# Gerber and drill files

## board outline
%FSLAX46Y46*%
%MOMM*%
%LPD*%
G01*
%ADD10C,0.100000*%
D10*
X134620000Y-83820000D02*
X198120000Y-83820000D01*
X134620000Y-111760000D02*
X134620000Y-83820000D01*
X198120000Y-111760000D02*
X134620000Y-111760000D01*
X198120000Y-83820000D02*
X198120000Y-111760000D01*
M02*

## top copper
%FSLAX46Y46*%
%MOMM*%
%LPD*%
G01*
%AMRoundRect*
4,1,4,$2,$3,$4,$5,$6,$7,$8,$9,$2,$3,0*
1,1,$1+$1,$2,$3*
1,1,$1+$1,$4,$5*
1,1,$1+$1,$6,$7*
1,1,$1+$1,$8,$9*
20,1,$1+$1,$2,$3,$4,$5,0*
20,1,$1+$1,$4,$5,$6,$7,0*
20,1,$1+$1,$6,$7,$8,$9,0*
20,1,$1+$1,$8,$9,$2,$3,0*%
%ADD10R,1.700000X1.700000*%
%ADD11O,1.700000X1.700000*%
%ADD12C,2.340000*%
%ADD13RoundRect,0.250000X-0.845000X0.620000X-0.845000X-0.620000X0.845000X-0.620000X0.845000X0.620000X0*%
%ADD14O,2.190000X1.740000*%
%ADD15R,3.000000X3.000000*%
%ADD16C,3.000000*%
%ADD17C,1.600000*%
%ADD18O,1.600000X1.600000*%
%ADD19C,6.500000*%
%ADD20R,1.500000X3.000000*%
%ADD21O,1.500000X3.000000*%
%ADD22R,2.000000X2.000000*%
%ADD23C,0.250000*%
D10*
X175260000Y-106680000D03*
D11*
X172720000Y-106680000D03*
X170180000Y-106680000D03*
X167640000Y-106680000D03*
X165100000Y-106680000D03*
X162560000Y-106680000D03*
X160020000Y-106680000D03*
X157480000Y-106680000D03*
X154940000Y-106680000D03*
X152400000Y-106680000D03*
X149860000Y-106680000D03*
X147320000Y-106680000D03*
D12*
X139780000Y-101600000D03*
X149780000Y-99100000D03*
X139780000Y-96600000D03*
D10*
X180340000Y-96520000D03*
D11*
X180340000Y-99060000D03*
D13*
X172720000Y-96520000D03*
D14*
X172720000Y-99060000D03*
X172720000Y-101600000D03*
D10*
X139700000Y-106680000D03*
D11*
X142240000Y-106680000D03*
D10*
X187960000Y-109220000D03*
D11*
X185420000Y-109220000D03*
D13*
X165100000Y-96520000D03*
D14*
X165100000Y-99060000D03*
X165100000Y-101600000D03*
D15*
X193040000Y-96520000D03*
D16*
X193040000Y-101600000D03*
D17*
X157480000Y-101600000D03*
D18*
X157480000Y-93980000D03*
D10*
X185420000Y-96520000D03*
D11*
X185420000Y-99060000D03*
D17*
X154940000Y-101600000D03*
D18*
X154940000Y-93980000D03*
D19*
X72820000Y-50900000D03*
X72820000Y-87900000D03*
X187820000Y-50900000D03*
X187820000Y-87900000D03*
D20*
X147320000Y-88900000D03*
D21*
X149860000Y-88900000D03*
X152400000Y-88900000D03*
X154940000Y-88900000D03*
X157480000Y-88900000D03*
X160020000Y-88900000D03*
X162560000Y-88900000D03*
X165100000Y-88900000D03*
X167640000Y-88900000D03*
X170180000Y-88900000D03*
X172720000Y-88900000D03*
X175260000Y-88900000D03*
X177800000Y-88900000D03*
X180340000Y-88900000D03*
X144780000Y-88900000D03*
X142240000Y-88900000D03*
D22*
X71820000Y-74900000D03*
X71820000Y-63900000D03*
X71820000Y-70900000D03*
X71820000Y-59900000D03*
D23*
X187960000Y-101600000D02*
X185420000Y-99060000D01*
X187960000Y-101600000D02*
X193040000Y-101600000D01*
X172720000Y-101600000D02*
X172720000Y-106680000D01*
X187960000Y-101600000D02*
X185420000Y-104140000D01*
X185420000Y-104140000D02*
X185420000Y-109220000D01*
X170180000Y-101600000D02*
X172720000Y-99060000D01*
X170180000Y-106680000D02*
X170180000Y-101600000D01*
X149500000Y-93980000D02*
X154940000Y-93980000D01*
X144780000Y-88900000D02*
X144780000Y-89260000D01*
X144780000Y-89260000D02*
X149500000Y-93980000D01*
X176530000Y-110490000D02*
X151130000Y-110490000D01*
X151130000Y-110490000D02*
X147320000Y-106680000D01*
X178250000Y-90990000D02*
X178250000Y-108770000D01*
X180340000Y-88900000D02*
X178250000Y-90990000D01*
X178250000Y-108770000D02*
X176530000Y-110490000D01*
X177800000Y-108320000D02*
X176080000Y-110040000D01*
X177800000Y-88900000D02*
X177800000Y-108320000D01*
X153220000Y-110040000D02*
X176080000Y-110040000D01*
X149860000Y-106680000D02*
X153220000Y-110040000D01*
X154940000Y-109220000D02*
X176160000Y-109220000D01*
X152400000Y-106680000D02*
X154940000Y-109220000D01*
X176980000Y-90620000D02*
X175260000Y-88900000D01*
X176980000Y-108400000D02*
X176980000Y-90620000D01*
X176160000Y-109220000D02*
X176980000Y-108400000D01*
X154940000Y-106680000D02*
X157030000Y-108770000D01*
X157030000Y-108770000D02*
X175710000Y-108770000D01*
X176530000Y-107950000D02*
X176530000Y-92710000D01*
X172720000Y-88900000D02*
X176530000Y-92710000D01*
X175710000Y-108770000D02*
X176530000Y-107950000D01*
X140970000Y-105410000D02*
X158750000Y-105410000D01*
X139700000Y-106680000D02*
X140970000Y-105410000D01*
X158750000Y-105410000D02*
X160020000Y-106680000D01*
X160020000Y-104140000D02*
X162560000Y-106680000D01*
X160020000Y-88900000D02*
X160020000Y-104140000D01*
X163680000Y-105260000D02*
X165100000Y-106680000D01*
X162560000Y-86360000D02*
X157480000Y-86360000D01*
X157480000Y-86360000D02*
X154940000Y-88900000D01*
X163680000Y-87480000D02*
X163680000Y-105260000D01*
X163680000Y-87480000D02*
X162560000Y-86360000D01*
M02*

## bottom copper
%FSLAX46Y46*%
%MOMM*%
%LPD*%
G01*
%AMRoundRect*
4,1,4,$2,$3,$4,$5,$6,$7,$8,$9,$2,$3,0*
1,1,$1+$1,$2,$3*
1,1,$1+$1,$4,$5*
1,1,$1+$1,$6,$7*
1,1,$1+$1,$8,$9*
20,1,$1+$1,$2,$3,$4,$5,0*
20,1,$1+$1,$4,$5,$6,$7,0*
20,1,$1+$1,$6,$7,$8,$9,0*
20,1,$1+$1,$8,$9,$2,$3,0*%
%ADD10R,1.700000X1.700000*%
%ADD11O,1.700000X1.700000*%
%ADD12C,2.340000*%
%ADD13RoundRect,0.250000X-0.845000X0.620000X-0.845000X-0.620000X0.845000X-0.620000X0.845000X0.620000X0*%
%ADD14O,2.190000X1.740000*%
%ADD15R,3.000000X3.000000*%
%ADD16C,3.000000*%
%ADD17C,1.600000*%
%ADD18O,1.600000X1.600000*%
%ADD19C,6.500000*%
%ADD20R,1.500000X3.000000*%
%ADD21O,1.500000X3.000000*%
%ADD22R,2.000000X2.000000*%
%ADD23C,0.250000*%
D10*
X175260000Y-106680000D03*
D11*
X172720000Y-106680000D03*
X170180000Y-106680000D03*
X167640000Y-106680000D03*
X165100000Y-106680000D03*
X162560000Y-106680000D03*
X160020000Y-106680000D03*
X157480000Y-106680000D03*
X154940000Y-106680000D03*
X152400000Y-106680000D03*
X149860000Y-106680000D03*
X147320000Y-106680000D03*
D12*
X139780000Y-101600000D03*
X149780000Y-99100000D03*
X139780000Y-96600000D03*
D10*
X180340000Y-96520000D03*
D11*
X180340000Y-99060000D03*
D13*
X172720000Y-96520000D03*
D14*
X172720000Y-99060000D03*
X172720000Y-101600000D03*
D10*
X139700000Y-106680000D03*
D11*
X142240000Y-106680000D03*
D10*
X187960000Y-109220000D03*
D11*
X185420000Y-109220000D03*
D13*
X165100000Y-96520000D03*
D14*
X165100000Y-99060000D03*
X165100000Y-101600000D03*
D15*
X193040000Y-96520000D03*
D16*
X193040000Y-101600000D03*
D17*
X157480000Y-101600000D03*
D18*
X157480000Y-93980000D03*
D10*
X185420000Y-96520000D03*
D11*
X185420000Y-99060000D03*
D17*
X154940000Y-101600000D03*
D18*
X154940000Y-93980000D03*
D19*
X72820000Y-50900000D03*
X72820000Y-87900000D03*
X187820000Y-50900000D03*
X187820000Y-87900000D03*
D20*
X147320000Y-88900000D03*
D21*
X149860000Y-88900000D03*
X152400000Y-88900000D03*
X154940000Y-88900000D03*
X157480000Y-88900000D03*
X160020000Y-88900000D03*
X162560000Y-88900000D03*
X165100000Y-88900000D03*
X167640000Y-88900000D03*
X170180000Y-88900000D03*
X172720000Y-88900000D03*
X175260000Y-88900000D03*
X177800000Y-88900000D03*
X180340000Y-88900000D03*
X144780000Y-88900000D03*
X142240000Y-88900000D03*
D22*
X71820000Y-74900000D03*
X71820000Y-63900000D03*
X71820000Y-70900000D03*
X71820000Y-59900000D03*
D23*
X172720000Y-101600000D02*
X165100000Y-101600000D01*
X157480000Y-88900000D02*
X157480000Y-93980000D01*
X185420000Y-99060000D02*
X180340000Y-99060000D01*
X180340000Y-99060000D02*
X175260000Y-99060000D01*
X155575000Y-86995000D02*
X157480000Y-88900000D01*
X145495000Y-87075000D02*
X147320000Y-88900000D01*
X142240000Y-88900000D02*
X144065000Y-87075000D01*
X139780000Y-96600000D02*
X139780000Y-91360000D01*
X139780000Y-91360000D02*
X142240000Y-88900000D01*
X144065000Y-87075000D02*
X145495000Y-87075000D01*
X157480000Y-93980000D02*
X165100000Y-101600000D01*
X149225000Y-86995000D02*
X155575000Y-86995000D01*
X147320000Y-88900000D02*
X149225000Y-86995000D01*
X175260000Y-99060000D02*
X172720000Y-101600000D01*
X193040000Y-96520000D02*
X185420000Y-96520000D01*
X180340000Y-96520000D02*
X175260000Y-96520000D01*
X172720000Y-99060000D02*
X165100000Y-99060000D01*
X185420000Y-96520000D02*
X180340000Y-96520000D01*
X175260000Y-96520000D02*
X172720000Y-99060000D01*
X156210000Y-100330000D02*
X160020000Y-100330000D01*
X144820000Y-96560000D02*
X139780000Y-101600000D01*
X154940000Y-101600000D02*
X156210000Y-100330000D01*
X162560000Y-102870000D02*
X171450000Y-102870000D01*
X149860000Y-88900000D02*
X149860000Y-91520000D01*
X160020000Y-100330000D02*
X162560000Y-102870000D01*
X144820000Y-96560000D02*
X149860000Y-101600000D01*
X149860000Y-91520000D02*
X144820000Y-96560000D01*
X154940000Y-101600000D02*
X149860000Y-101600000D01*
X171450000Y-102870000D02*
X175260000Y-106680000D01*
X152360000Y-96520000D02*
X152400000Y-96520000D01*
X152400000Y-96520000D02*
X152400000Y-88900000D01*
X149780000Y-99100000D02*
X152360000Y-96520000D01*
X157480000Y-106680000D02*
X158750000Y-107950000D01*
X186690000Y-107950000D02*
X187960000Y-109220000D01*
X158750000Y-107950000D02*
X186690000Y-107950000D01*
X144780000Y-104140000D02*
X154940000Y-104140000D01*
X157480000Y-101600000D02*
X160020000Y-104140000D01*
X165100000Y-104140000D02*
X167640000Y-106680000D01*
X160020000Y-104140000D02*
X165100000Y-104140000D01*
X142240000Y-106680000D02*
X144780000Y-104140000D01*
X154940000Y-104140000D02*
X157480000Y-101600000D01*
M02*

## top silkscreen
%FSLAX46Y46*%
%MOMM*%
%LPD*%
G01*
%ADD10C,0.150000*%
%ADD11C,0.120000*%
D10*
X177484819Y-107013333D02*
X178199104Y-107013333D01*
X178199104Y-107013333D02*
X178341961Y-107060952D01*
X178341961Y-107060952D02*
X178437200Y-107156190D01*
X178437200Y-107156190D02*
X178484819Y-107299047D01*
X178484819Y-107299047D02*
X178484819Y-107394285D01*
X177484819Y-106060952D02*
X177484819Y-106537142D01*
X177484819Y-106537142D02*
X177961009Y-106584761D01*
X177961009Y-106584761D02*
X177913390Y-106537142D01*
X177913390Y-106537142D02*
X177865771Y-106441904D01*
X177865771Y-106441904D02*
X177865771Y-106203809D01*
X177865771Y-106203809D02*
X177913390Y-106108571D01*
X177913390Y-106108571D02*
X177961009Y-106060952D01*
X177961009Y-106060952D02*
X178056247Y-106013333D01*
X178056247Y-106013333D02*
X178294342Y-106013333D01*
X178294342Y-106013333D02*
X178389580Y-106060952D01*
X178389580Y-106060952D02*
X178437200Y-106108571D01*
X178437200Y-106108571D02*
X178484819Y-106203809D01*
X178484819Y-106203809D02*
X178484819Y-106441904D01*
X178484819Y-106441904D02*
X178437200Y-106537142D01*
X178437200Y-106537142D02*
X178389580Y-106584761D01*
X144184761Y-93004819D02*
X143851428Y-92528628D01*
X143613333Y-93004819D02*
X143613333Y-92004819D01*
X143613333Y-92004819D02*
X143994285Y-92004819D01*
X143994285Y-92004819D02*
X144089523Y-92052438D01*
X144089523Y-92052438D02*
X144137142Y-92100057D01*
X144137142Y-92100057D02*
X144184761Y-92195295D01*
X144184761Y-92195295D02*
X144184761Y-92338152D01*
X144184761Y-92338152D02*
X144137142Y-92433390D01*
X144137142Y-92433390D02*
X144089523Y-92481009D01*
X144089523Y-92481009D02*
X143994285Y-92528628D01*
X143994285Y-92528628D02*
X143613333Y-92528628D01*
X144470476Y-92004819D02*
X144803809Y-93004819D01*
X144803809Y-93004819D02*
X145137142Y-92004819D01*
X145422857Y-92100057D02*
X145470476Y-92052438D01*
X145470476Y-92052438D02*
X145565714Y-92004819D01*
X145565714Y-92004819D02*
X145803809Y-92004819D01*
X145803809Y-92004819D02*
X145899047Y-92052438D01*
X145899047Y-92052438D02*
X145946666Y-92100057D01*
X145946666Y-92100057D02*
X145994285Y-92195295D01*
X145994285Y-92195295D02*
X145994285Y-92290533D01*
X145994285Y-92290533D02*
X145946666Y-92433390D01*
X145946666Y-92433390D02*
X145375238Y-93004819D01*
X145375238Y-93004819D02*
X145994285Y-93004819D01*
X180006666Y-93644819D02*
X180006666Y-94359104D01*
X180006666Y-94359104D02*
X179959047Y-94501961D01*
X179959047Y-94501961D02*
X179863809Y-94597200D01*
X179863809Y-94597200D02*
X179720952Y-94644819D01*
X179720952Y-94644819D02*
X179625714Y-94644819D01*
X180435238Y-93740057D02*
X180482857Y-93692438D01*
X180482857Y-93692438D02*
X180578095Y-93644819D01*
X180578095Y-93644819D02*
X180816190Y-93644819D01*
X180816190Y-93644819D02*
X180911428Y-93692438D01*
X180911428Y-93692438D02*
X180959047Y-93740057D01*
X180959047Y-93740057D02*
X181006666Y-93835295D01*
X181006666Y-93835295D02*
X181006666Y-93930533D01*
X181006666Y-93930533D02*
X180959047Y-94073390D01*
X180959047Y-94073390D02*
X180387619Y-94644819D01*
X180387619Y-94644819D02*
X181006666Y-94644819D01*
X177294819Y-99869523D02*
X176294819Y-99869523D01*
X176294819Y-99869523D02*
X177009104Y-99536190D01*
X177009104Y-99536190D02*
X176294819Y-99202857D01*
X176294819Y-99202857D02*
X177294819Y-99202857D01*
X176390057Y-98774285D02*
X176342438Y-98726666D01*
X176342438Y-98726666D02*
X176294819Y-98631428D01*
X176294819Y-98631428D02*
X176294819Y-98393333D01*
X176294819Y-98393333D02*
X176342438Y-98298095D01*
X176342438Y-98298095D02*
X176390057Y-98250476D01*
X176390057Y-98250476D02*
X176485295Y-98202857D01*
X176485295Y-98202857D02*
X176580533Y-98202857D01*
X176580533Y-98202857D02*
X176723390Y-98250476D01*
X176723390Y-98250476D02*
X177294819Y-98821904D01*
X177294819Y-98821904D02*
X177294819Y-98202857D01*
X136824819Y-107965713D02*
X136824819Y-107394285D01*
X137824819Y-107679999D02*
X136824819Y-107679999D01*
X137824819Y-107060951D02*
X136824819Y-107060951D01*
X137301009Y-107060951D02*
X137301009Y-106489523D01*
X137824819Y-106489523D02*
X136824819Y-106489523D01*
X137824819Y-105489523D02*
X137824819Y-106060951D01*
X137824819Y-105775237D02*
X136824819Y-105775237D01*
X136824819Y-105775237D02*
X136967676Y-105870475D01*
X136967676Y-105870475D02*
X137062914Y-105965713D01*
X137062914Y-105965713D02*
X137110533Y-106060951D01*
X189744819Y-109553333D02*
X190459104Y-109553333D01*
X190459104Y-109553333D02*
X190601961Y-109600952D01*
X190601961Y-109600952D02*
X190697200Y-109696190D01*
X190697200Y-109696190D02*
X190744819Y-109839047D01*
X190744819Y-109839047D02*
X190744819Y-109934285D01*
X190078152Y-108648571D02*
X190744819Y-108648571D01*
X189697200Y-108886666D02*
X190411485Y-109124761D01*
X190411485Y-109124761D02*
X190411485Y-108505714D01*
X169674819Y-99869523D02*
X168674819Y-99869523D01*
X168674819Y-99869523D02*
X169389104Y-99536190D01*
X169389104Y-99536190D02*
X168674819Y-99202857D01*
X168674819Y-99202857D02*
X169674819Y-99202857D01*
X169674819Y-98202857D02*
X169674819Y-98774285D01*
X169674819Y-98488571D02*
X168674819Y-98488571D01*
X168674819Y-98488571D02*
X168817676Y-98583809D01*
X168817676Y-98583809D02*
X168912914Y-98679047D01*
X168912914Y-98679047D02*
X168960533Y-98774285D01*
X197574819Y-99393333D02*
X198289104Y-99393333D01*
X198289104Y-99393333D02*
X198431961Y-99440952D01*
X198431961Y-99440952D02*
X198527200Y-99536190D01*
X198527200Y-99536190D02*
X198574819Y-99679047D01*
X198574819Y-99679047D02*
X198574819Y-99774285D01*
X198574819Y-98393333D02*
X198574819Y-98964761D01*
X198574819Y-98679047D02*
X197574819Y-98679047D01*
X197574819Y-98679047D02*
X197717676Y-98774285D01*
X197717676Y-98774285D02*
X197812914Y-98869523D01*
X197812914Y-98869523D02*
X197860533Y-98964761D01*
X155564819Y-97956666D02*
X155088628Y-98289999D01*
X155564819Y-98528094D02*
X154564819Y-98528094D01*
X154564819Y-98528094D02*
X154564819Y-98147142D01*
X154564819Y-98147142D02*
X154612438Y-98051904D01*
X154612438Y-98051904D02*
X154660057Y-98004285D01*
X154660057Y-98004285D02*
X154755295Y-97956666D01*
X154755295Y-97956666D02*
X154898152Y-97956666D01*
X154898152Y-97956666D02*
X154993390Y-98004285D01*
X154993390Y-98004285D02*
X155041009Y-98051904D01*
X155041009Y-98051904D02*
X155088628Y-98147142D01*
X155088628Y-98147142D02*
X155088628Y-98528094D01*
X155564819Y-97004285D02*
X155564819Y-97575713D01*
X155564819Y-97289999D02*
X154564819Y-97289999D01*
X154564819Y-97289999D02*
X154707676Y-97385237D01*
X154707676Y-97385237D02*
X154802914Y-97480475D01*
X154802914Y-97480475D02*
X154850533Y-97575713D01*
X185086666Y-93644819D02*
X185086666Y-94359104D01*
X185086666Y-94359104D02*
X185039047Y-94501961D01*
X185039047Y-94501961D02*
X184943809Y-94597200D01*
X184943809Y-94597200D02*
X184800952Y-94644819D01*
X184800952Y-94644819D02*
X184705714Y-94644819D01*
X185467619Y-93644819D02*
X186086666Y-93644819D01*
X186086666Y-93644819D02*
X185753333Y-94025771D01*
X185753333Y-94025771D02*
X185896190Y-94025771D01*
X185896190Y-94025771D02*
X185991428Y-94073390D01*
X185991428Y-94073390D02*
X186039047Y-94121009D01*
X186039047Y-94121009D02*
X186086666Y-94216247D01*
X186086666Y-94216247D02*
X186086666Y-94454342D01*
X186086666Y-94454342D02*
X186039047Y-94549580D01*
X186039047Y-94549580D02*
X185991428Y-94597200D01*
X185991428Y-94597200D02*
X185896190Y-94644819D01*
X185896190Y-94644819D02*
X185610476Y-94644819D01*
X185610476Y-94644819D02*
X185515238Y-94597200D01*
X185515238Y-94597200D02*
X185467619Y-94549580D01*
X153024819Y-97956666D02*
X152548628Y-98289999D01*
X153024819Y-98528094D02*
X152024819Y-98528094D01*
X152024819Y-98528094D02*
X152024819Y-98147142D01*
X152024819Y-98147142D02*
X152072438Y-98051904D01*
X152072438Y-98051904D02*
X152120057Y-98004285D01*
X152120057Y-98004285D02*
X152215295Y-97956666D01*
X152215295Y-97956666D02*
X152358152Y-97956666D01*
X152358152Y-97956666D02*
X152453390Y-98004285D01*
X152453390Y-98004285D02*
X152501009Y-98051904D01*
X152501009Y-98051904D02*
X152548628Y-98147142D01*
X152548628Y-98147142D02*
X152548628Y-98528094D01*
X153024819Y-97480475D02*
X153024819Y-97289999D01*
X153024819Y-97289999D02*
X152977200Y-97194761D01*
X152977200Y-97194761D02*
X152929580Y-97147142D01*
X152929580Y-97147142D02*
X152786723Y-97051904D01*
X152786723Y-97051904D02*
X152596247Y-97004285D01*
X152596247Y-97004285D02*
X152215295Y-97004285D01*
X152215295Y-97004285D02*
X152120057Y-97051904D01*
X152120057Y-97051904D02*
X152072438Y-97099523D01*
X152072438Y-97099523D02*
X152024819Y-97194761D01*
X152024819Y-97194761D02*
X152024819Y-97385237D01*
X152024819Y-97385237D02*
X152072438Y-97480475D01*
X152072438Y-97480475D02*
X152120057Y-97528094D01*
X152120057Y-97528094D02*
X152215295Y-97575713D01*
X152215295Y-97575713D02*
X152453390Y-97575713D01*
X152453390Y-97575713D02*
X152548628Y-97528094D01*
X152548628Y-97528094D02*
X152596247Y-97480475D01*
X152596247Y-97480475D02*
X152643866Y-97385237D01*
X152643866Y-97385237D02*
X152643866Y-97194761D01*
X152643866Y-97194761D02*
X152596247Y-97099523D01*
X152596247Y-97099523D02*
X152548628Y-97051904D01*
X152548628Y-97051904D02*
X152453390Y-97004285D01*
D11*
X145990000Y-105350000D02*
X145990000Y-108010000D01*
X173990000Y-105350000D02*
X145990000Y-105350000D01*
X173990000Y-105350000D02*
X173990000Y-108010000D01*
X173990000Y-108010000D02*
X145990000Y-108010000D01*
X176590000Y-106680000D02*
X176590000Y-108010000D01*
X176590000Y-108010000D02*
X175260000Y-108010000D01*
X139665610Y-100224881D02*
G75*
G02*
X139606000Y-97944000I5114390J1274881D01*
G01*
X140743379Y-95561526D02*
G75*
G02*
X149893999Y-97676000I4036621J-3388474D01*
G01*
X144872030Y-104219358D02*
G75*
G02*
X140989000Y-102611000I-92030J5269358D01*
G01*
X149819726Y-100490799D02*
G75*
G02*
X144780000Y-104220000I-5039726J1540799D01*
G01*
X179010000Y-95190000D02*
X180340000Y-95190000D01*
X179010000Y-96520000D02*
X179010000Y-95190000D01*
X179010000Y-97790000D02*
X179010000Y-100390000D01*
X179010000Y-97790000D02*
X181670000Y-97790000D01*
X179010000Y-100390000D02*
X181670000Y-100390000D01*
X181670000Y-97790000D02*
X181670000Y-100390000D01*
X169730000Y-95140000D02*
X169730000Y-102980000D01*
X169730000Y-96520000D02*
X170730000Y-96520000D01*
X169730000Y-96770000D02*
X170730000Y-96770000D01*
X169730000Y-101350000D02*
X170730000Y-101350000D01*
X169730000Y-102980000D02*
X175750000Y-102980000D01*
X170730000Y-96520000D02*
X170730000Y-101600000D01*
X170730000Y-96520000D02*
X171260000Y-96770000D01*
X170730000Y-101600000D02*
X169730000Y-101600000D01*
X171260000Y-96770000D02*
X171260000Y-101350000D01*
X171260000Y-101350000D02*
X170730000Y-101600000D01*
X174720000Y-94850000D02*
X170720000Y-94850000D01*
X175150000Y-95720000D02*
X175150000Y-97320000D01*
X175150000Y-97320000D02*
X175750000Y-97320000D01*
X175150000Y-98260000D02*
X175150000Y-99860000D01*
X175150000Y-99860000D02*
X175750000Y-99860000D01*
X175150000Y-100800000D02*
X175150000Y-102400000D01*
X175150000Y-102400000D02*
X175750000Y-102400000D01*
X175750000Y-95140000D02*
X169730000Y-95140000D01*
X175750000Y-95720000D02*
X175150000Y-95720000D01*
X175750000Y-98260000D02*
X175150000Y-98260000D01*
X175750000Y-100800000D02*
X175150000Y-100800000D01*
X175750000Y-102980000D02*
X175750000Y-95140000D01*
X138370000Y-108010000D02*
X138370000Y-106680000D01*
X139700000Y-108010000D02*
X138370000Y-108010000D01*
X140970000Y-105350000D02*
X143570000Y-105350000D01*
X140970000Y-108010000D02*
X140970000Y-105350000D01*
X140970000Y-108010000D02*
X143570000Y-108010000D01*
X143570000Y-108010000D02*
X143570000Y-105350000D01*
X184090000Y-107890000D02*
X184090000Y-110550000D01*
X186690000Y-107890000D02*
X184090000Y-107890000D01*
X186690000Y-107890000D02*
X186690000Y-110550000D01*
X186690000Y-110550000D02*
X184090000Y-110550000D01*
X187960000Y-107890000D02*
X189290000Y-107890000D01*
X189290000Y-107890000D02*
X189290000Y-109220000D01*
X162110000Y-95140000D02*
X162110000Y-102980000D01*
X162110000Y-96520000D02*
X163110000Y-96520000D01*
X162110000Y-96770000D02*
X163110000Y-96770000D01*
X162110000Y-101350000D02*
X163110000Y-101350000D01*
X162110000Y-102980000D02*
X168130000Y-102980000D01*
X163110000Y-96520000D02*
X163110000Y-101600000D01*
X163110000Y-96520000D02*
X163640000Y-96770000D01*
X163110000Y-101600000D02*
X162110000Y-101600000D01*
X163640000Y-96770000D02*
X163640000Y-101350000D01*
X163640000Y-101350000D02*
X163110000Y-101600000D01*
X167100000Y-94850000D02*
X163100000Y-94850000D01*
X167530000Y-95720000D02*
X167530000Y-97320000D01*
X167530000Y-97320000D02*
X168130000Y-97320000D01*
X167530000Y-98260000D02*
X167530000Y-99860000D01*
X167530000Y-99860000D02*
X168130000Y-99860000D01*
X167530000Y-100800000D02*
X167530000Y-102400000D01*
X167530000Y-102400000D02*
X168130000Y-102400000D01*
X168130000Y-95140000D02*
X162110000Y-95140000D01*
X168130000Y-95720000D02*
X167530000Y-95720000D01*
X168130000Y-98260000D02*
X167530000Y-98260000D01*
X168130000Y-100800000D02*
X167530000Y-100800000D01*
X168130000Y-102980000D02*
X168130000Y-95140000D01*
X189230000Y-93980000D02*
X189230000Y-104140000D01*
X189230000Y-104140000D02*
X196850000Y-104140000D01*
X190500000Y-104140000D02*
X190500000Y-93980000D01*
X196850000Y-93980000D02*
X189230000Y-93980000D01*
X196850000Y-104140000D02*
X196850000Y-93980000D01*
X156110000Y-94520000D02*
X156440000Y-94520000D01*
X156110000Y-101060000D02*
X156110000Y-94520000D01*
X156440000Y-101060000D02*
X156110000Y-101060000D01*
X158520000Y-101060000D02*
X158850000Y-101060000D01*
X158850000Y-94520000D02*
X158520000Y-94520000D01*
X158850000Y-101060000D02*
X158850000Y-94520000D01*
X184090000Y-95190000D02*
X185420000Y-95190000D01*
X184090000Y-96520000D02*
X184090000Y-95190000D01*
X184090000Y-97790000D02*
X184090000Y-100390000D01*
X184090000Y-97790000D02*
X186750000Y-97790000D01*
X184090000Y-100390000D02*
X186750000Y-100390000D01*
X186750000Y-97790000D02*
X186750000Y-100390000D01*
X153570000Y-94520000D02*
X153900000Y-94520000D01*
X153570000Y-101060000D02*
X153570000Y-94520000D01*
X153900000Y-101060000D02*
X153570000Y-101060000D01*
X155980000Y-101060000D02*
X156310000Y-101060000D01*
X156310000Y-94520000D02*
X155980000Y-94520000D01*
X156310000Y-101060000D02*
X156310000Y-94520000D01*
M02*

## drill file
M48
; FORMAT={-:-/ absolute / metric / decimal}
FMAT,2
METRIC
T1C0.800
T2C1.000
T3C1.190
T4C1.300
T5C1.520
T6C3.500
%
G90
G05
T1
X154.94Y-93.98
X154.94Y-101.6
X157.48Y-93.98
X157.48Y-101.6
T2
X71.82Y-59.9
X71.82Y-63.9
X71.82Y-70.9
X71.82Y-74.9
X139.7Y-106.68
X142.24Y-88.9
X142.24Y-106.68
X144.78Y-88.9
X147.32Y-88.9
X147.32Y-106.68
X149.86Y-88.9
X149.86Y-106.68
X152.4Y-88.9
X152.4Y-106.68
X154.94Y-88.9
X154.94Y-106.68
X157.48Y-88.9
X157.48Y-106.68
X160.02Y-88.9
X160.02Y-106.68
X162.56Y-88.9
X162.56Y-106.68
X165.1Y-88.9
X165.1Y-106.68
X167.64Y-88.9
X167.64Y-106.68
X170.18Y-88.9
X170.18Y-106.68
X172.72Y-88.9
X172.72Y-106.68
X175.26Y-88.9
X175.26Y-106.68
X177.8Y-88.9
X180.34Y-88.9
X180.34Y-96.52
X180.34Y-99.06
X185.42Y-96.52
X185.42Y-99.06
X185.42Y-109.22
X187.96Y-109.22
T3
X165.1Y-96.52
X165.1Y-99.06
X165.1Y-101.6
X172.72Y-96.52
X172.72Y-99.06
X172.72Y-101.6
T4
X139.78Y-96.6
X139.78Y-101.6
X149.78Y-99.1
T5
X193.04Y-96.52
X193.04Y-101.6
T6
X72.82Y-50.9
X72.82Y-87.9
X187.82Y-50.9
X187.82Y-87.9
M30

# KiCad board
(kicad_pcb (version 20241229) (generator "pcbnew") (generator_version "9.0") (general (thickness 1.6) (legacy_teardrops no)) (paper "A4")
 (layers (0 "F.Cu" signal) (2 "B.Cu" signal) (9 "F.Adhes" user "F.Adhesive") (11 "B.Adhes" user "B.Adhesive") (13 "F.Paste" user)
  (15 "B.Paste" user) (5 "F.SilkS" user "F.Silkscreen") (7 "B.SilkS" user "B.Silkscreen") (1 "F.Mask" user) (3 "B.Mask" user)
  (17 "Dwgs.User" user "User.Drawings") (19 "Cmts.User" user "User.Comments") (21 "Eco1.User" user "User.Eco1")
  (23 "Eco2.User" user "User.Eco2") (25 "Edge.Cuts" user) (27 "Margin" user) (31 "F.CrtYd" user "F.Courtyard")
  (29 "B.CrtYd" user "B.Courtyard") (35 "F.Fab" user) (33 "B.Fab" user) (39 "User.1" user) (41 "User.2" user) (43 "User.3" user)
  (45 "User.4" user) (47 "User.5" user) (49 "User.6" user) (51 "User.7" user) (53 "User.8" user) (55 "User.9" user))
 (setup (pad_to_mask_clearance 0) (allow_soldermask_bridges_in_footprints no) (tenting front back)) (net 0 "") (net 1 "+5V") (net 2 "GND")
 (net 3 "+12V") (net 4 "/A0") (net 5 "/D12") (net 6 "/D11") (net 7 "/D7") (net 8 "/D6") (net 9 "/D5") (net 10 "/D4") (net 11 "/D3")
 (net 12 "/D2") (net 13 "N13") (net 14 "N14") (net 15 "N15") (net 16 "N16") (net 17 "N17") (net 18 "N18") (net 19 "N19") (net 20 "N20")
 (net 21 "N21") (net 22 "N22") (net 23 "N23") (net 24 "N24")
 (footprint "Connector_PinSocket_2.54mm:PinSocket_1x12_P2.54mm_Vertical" (layer "F.Cu") (at 175.26 106.68 -90)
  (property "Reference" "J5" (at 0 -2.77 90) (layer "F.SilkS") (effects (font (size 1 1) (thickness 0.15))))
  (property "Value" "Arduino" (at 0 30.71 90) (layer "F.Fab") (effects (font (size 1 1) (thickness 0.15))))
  (fp_line (start -1.33 29.27) (end 1.33 29.27) (stroke (width 0.12) (type solid)) (layer "F.SilkS"))
  (fp_line (start -1.33 1.27) (end -1.33 29.27) (stroke (width 0.12) (type solid)) (layer "F.SilkS"))
  (fp_line (start -1.33 1.27) (end 1.33 1.27) (stroke (width 0.12) (type solid)) (layer "F.SilkS"))
  (fp_line (start 1.33 1.27) (end 1.33 29.27) (stroke (width 0.12) (type solid)) (layer "F.SilkS"))
  (fp_line (start 0 -1.33) (end 1.33 -1.33) (stroke (width 0.12) (type solid)) (layer "F.SilkS"))
  (fp_line (start 1.33 -1.33) (end 1.33 0) (stroke (width 0.12) (type solid)) (layer "F.SilkS"))
  (pad "1" thru_hole rect (at 0 0 270) (size 1.7 1.7) (drill 1) (layers "*.Cu" "*.Mask") (remove_unused_layers no) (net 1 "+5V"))
  (pad "2" thru_hole oval (at 0 2.54 270) (size 1.7 1.7) (drill 1) (layers "*.Cu" "*.Mask") (remove_unused_layers no) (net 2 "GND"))
  (pad "3" thru_hole oval (at 0 5.08 270) (size 1.7 1.7) (drill 1) (layers "*.Cu" "*.Mask") (remove_unused_layers no) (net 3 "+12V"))
  (pad "4" thru_hole oval (at 0 7.62 270) (size 1.7 1.7) (drill 1) (layers "*.Cu" "*.Mask") (remove_unused_layers no) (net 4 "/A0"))
  (pad "5" thru_hole oval (at 0 10.16 270) (size 1.7 1.7) (drill 1) (layers "*.Cu" "*.Mask") (remove_unused_layers no) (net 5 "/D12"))
  (pad "6" thru_hole oval (at 0 12.7 270) (size 1.7 1.7) (drill 1) (layers "*.Cu" "*.Mask") (remove_unused_layers no) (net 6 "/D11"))
  (pad "7" thru_hole oval (at 0 15.24 270) (size 1.7 1.7) (drill 1) (layers "*.Cu" "*.Mask") (remove_unused_layers no) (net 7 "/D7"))
  (pad "8" thru_hole oval (at 0 17.78 270) (size 1.7 1.7) (drill 1) (layers "*.Cu" "*.Mask") (remove_unused_layers no) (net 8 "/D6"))
  (pad "9" thru_hole oval (at 0 20.32 270) (size 1.7 1.7) (drill 1) (layers "*.Cu" "*.Mask") (remove_unused_layers no) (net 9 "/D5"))
  (pad "10" thru_hole oval (at 0 22.86 270) (size 1.7 1.7) (drill 1) (layers "*.Cu" "*.Mask") (remove_unused_layers no) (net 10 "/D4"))
  (pad "11" thru_hole oval (at 0 25.4 270) (size 1.7 1.7) (drill 1) (layers "*.Cu" "*.Mask") (remove_unused_layers no) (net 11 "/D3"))
  (pad "12" thru_hole oval (at 0 27.94 270) (size 1.7 1.7) (drill 1) (layers "*.Cu" "*.Mask") (remove_unused_layers no) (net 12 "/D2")))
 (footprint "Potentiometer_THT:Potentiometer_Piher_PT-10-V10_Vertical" (layer "F.Cu") (at 139.78 101.6)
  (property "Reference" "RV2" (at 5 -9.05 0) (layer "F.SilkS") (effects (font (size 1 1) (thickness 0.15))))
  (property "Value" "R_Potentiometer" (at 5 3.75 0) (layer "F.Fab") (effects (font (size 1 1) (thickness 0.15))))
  (fp_arc (start -0.11439 -1.375119) (mid -0.269093 -2.512295) (end -0.174 -3.656) (stroke (width 0.12) (type solid)) (layer "F.SilkS"))
  (fp_arc (start 0.963379 -6.038474) (mid 6.186565 -7.784991) (end 10.114 -3.924) (stroke (width 0.12) (type solid)) (layer "F.SilkS"))
  (fp_arc (start 5.09203 2.619358) (mid 2.983245 2.219015) (end 1.209 1.011) (stroke (width 0.12) (type solid)) (layer "F.SilkS"))
  (fp_arc (start 10.039726 -1.109201) (mid 8.134716 1.586326) (end 5 2.62) (stroke (width 0.12) (type solid)) (layer "F.SilkS"))
  (pad "1" thru_hole circle (at 0 0) (size 2.34 2.34) (drill 1.3) (layers "*.Cu" "*.Mask") (remove_unused_layers no) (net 1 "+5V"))
  (pad "2" thru_hole circle (at 10 -2.5) (size 2.34 2.34) (drill 1.3) (layers "*.Cu" "*.Mask") (remove_unused_layers no) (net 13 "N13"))
  (pad "3" thru_hole circle (at 0 -5) (size 2.34 2.34) (drill 1.3) (layers "*.Cu" "*.Mask") (remove_unused_layers no) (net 2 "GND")))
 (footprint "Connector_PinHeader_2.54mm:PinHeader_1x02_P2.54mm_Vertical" (layer "F.Cu") (at 180.34 96.52)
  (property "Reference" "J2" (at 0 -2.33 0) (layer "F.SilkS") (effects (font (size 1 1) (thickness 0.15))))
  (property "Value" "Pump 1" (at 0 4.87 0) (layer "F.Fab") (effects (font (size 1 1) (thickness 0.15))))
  (fp_line (start -1.33 -1.33) (end 0 -1.33) (stroke (width 0.12) (type solid)) (layer "F.SilkS"))
  (fp_line (start -1.33 0) (end -1.33 -1.33) (stroke (width 0.12) (type solid)) (layer "F.SilkS"))
  (fp_line (start -1.33 1.27) (end -1.33 3.87) (stroke (width 0.12) (type solid)) (layer "F.SilkS"))
  (fp_line (start -1.33 1.27) (end 1.33 1.27) (stroke (width 0.12) (type solid)) (layer "F.SilkS"))
  (fp_line (start -1.33 3.87) (end 1.33 3.87) (stroke (width 0.12) (type solid)) (layer "F.SilkS"))
  (fp_line (start 1.33 1.27) (end 1.33 3.87) (stroke (width 0.12) (type solid)) (layer "F.SilkS"))
  (pad "1" thru_hole rect (at 0 0) (size 1.7 1.7) (drill 1) (layers "*.Cu" "*.Mask") (remove_unused_layers no) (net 3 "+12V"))
  (pad "2" thru_hole oval (at 0 2.54) (size 1.7 1.7) (drill 1) (layers "*.Cu" "*.Mask") (remove_unused_layers no) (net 2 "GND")))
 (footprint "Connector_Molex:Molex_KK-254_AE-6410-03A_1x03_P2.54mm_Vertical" (layer "F.Cu") (at 172.72 96.52 -90)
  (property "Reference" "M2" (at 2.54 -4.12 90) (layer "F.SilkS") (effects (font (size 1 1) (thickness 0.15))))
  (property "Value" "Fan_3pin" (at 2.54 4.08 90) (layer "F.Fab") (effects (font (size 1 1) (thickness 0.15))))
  (fp_line (start -1.38 2.99) (end 6.46 2.99) (stroke (width 0.12) (type solid)) (layer "F.SilkS"))
  (fp_line (start 0 2.99) (end 0 1.99) (stroke (width 0.12) (type solid)) (layer "F.SilkS"))
  (fp_line (start 0.25 2.99) (end 0.25 1.99) (stroke (width 0.12) (type solid)) (layer "F.SilkS"))
  (fp_line (start 4.83 2.99) (end 4.83 1.99) (stroke (width 0.12) (type solid)) (layer "F.SilkS"))
  (fp_line (start 6.46 2.99) (end 6.46 -3.03) (stroke (width 0.12) (type solid)) (layer "F.SilkS"))
  (fp_line (start 0 1.99) (end 5.08 1.99) (stroke (width 0.12) (type solid)) (layer "F.SilkS"))
  (fp_line (start 0 1.99) (end 0.25 1.46) (stroke (width 0.12) (type solid)) (layer "F.SilkS"))
  (fp_line (start 5.08 1.99) (end 5.08 2.99) (stroke (width 0.12) (type solid)) (layer "F.SilkS"))
  (fp_line (start 0.25 1.46) (end 4.83 1.46) (stroke (width 0.12) (type solid)) (layer "F.SilkS"))
  (fp_line (start 4.83 1.46) (end 5.08 1.99) (stroke (width 0.12) (type solid)) (layer "F.SilkS"))
  (fp_line (start -1.67 -2) (end -1.67 2) (stroke (width 0.12) (type solid)) (layer "F.SilkS"))
  (fp_line (start -0.8 -2.43) (end 0.8 -2.43) (stroke (width 0.12) (type solid)) (layer "F.SilkS"))
  (fp_line (start 0.8 -2.43) (end 0.8 -3.03) (stroke (width 0.12) (type solid)) (layer "F.SilkS"))
  (fp_line (start 1.74 -2.43) (end 3.34 -2.43) (stroke (width 0.12) (type solid)) (layer "F.SilkS"))
  (fp_line (start 3.34 -2.43) (end 3.34 -3.03) (stroke (width 0.12) (type solid)) (layer "F.SilkS"))
  (fp_line (start 4.28 -2.43) (end 5.88 -2.43) (stroke (width 0.12) (type solid)) (layer "F.SilkS"))
  (fp_line (start 5.88 -2.43) (end 5.88 -3.03) (stroke (width 0.12) (type solid)) (layer "F.SilkS"))
  (fp_line (start -1.38 -3.03) (end -1.38 2.99) (stroke (width 0.12) (type solid)) (layer "F.SilkS"))
  (fp_line (start -0.8 -3.03) (end -0.8 -2.43) (stroke (width 0.12) (type solid)) (layer "F.SilkS"))
  (fp_line (start 1.74 -3.03) (end 1.74 -2.43) (stroke (width 0.12) (type solid)) (layer "F.SilkS"))
  (fp_line (start 4.28 -3.03) (end 4.28 -2.43) (stroke (width 0.12) (type solid)) (layer "F.SilkS"))
  (fp_line (start 6.46 -3.03) (end -1.38 -3.03) (stroke (width 0.12) (type solid)) (layer "F.SilkS"))
  (pad "1" thru_hole roundrect (at 0 0 270) (size 1.74 2.19) (drill 1.19) (layers "*.Cu" "*.Mask") (remove_unused_layers no)
   (roundrect_rratio 0.143678) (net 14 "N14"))
  (pad "2" thru_hole oval (at 2.54 0 270) (size 1.74 2.19) (drill 1.19) (layers "*.Cu" "*.Mask") (remove_unused_layers no) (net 3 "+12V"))
  (pad "3" thru_hole oval (at 5.08 0 270) (size 1.74 2.19) (drill 1.19) (layers "*.Cu" "*.Mask") (remove_unused_layers no) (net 2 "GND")))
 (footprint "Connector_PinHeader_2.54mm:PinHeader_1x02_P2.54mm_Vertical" (layer "F.Cu") (at 139.7 106.68 90)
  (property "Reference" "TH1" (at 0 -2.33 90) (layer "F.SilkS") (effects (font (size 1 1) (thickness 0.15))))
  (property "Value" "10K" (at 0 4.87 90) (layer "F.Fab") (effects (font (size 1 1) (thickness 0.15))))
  (fp_line (start -1.33 -1.33) (end 0 -1.33) (stroke (width 0.12) (type solid)) (layer "F.SilkS"))
  (fp_line (start -1.33 0) (end -1.33 -1.33) (stroke (width 0.12) (type solid)) (layer "F.SilkS"))
  (fp_line (start 1.33 1.27) (end 1.33 3.87) (stroke (width 0.12) (type solid)) (layer "F.SilkS"))
  (fp_line (start -1.33 1.27) (end 1.33 1.27) (stroke (width 0.12) (type solid)) (layer "F.SilkS"))
  (fp_line (start -1.33 1.27) (end -1.33 3.87) (stroke (width 0.12) (type solid)) (layer "F.SilkS"))
  (fp_line (start -1.33 3.87) (end 1.33 3.87) (stroke (width 0.12) (type solid)) (layer "F.SilkS"))
  (pad "1" thru_hole rect (at 0 0 90) (size 1.7 1.7) (drill 1) (layers "*.Cu" "*.Mask") (remove_unused_layers no) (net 7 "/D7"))
  (pad "2" thru_hole oval (at 0 2.54 90) (size 1.7 1.7) (drill 1) (layers "*.Cu" "*.Mask") (remove_unused_layers no) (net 4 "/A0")))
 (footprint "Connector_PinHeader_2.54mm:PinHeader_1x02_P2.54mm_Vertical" (layer "F.Cu") (at 187.96 109.22 -90)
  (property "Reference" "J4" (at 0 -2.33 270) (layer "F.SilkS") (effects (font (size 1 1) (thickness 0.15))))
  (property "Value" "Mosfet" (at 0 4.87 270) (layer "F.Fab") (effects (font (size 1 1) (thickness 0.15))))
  (fp_line (start -1.33 3.87) (end 1.33 3.87) (stroke (width 0.12) (type solid)) (layer "F.SilkS"))
  (fp_line (start -1.33 1.27) (end -1.33 3.87) (stroke (width 0.12) (type solid)) (layer "F.SilkS"))
  (fp_line (start -1.33 1.27) (end 1.33 1.27) (stroke (width 0.12) (type solid)) (layer "F.SilkS"))
  (fp_line (start 1.33 1.27) (end 1.33 3.87) (stroke (width 0.12) (type solid)) (layer "F.SilkS"))
  (fp_line (start -1.33 0) (end -1.33 -1.33) (stroke (width 0.12) (type solid)) (layer "F.SilkS"))
  (fp_line (start -1.33 -1.33) (end 0 -1.33) (stroke (width 0.12) (type solid)) (layer "F.SilkS"))
  (pad "1" thru_hole rect (at 0 0 270) (size 1.7 1.7) (drill 1) (layers "*.Cu" "*.Mask") (remove_unused_layers no) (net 8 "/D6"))
  (pad "2" thru_hole oval (at 0 2.54 270) (size 1.7 1.7) (drill 1) (layers "*.Cu" "*.Mask") (remove_unused_layers no) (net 2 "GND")))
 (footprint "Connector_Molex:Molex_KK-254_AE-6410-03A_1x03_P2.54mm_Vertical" (layer "F.Cu") (at 165.1 96.52 -90)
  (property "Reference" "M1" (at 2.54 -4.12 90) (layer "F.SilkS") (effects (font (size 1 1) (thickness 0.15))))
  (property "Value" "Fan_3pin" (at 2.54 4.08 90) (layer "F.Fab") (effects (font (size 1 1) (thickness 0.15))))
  (fp_line (start -1.38 2.99) (end 6.46 2.99) (stroke (width 0.12) (type solid)) (layer "F.SilkS"))
  (fp_line (start 0 2.99) (end 0 1.99) (stroke (width 0.12) (type solid)) (layer "F.SilkS"))
  (fp_line (start 0.25 2.99) (end 0.25 1.99) (stroke (width 0.12) (type solid)) (layer "F.SilkS"))
  (fp_line (start 4.83 2.99) (end 4.83 1.99) (stroke (width 0.12) (type solid)) (layer "F.SilkS"))
  (fp_line (start 6.46 2.99) (end 6.46 -3.03) (stroke (width 0.12) (type solid)) (layer "F.SilkS"))
  (fp_line (start 0 1.99) (end 5.08 1.99) (stroke (width 0.12) (type solid)) (layer "F.SilkS"))
  (fp_line (start 0 1.99) (end 0.25 1.46) (stroke (width 0.12) (type solid)) (layer "F.SilkS"))
  (fp_line (start 5.08 1.99) (end 5.08 2.99) (stroke (width 0.12) (type solid)) (layer "F.SilkS"))
  (fp_line (start 0.25 1.46) (end 4.83 1.46) (stroke (width 0.12) (type solid)) (layer "F.SilkS"))
  (fp_line (start 4.83 1.46) (end 5.08 1.99) (stroke (width 0.12) (type solid)) (layer "F.SilkS"))
  (fp_line (start -1.67 -2) (end -1.67 2) (stroke (width 0.12) (type solid)) (layer "F.SilkS"))
  (fp_line (start -0.8 -2.43) (end 0.8 -2.43) (stroke (width 0.12) (type solid)) (layer "F.SilkS"))
  (fp_line (start 0.8 -2.43) (end 0.8 -3.03) (stroke (width 0.12) (type solid)) (layer "F.SilkS"))
  (fp_line (start 1.74 -2.43) (end 3.34 -2.43) (stroke (width 0.12) (type solid)) (layer "F.SilkS"))
  (fp_line (start 3.34 -2.43) (end 3.34 -3.03) (stroke (width 0.12) (type solid)) (layer "F.SilkS"))
  (fp_line (start 4.28 -2.43) (end 5.88 -2.43) (stroke (width 0.12) (type solid)) (layer "F.SilkS"))
  (fp_line (start 5.88 -2.43) (end 5.88 -3.03) (stroke (width 0.12) (type solid)) (layer "F.SilkS"))
  (fp_line (start -1.38 -3.03) (end -1.38 2.99) (stroke (width 0.12) (type solid)) (layer "F.SilkS"))
  (fp_line (start -0.8 -3.03) (end -0.8 -2.43) (stroke (width 0.12) (type solid)) (layer "F.SilkS"))
  (fp_line (start 1.74 -3.03) (end 1.74 -2.43) (stroke (width 0.12) (type solid)) (layer "F.SilkS"))
  (fp_line (start 4.28 -3.03) (end 4.28 -2.43) (stroke (width 0.12) (type solid)) (layer "F.SilkS"))
  (fp_line (start 6.46 -3.03) (end -1.38 -3.03) (stroke (width 0.12) (type solid)) (layer "F.SilkS"))
  (pad "1" thru_hole roundrect (at 0 0 270) (size 1.74 2.19) (drill 1.19) (layers "*.Cu" "*.Mask") (remove_unused_layers no)
   (roundrect_rratio 0.143678) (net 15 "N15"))
  (pad "2" thru_hole oval (at 2.54 0 270) (size 1.74 2.19) (drill 1.19) (layers "*.Cu" "*.Mask") (remove_unused_layers no) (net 3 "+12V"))
  (pad "3" thru_hole oval (at 5.08 0 270) (size 1.74 2.19) (drill 1.19) (layers "*.Cu" "*.Mask") (remove_unused_layers no) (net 2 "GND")))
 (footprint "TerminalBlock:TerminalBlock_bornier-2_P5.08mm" (layer "F.Cu") (at 193.04 96.52 -90)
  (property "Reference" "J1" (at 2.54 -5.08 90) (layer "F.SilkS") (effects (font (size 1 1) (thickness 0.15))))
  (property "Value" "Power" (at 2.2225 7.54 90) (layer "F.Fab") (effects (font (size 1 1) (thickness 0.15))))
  (fp_line (start -2.54 3.81) (end 7.62 3.81) (stroke (width 0.12) (type solid)) (layer "F.SilkS"))
  (fp_line (start 7.62 3.81) (end 7.62 -3.81) (stroke (width 0.12) (type solid)) (layer "F.SilkS"))
  (fp_line (start 7.62 2.54) (end -2.54 2.54) (stroke (width 0.12) (type solid)) (layer "F.SilkS"))
  (fp_line (start -2.54 -3.81) (end -2.54 3.81) (stroke (width 0.12) (type solid)) (layer "F.SilkS"))
  (fp_line (start 7.62 -3.81) (end -2.54 -3.81) (stroke (width 0.12) (type solid)) (layer "F.SilkS"))
  (pad "1" thru_hole rect (at 0 0 270) (size 3 3) (drill 1.52) (layers "*.Cu" "*.Mask") (remove_unused_layers no) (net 3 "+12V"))
  (pad "2" thru_hole circle (at 5.08 0 270) (size 3 3) (drill 1.52) (layers "*.Cu" "*.Mask") (remove_unused_layers no) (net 2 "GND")))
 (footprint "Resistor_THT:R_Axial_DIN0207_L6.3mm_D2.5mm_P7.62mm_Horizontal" (layer "F.Cu") (at 157.48 101.6 90)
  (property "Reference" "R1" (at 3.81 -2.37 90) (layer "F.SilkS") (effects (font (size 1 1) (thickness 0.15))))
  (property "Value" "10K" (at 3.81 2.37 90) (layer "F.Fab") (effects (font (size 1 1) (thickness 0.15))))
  (fp_line (start 7.08 -1.37) (end 7.08 -1.04) (stroke (width 0.12) (type solid)) (layer "F.SilkS"))
  (fp_line (start 0.54 -1.37) (end 7.08 -1.37) (stroke (width 0.12) (type solid)) (layer "F.SilkS"))
  (fp_line (start 0.54 -1.04) (end 0.54 -1.37) (stroke (width 0.12) (type solid)) (layer "F.SilkS"))
  (fp_line (start 0.54 1.04) (end 0.54 1.37) (stroke (width 0.12) (type solid)) (layer "F.SilkS"))
  (fp_line (start 7.08 1.37) (end 7.08 1.04) (stroke (width 0.12) (type solid)) (layer "F.SilkS"))
  (fp_line (start 0.54 1.37) (end 7.08 1.37) (stroke (width 0.12) (type solid)) (layer "F.SilkS"))
  (pad "1" thru_hole circle (at 0 0 90) (size 1.6 1.6) (drill 0.8) (layers "*.Cu" "*.Mask") (remove_unused_layers no) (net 4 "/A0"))
  (pad "2" thru_hole oval (at 7.62 0 90) (size 1.6 1.6) (drill 0.8) (layers "*.Cu" "*.Mask") (remove_unused_layers no) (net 2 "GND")))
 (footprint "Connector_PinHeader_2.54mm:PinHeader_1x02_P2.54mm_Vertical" (layer "F.Cu") (at 185.42 96.52)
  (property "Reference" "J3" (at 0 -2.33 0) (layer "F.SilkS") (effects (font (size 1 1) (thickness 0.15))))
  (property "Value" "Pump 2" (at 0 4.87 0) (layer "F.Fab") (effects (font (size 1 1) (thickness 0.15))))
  (fp_line (start -1.33 -1.33) (end 0 -1.33) (stroke (width 0.12) (type solid)) (layer "F.SilkS"))
  (fp_line (start -1.33 0) (end -1.33 -1.33) (stroke (width 0.12) (type solid)) (layer "F.SilkS"))
  (fp_line (start -1.33 1.27) (end -1.33 3.87) (stroke (width 0.12) (type solid)) (layer "F.SilkS"))
  (fp_line (start -1.33 1.27) (end 1.33 1.27) (stroke (width 0.12) (type solid)) (layer "F.SilkS"))
  (fp_line (start -1.33 3.87) (end 1.33 3.87) (stroke (width 0.12) (type solid)) (layer "F.SilkS"))
  (fp_line (start 1.33 1.27) (end 1.33 3.87) (stroke (width 0.12) (type solid)) (layer "F.SilkS"))
  (pad "1" thru_hole rect (at 0 0) (size 1.7 1.7) (drill 1) (layers "*.Cu" "*.Mask") (remove_unused_layers no) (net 3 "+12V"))
  (pad "2" thru_hole oval (at 0 2.54) (size 1.7 1.7) (drill 1) (layers "*.Cu" "*.Mask") (remove_unused_layers no) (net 2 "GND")))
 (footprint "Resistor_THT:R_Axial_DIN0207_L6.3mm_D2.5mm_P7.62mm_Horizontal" (layer "F.Cu") (at 154.94 101.6 90)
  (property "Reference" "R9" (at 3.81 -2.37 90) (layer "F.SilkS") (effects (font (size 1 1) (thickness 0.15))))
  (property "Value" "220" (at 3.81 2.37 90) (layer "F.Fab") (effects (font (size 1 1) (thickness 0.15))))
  (fp_line (start 7.08 -1.37) (end 7.08 -1.04) (stroke (width 0.12) (type solid)) (layer "F.SilkS"))
  (fp_line (start 0.54 -1.37) (end 7.08 -1.37) (stroke (width 0.12) (type solid)) (layer "F.SilkS"))
  (fp_line (start 0.54 -1.04) (end 0.54 -1.37) (stroke (width 0.12) (type solid)) (layer "F.SilkS"))
  (fp_line (start 0.54 1.04) (end 0.54 1.37) (stroke (width 0.12) (type solid)) (layer "F.SilkS"))
  (fp_line (start 7.08 1.37) (end 7.08 1.04) (stroke (width 0.12) (type solid)) (layer "F.SilkS"))
  (fp_line (start 0.54 1.37) (end 7.08 1.37) (stroke (width 0.12) (type solid)) (layer "F.SilkS"))
  (pad "1" thru_hole circle (at 0 0 90) (size 1.6 1.6) (drill 0.8) (layers "*.Cu" "*.Mask") (remove_unused_layers no) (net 1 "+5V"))
  (pad "2" thru_hole oval (at 7.62 0 90) (size 1.6 1.6) (drill 0.8) (layers "*.Cu" "*.Mask") (remove_unused_layers no) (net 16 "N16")))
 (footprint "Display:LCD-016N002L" (layer "B.Cu") (at 147.32 88.9)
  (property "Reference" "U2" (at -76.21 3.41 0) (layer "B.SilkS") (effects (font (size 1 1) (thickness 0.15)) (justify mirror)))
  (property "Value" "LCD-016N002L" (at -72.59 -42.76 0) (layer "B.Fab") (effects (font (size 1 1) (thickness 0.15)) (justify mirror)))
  (pad "" thru_hole circle (at -74.5 -38 180) (size 6.5 6.5) (drill 3.5) (layers "*.Cu" "*.Mask") (remove_unused_layers no))
  (pad "" thru_hole circle (at -74.5 -1 180) (size 6.5 6.5) (drill 3.5) (layers "*.Cu" "*.Mask") (remove_unused_layers no))
  (pad "" thru_hole circle (at 40.5 -38 180) (size 6.5 6.5) (drill 3.5) (layers "*.Cu" "*.Mask") (remove_unused_layers no))
  (pad "" thru_hole circle (at 40.5 -1 180) (size 6.5 6.5) (drill 3.5) (layers "*.Cu" "*.Mask") (remove_unused_layers no))
  (pad "1" thru_hole rect (at 0 0 180) (size 1.5 3) (drill 1) (layers "*.Cu" "*.Mask") (remove_unused_layers no) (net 2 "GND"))
  (pad "2" thru_hole oval (at 2.54 0 180) (size 1.5 3) (drill 1) (layers "*.Cu" "*.Mask") (remove_unused_layers no) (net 1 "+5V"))
  (pad "3" thru_hole oval (at 5.08 0 180) (size 1.5 3) (drill 1) (layers "*.Cu" "*.Mask") (remove_unused_layers no) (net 13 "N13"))
  (pad "4" thru_hole oval (at 7.62 0 180) (size 1.5 3) (drill 1) (layers "*.Cu" "*.Mask") (remove_unused_layers no) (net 5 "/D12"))
  (pad "5" thru_hole oval (at 10.16 0 180) (size 1.5 3) (drill 1) (layers "*.Cu" "*.Mask") (remove_unused_layers no) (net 2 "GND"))
  (pad "6" thru_hole oval (at 12.7 0 180) (size 1.5 3) (drill 1) (layers "*.Cu" "*.Mask") (remove_unused_layers no) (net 6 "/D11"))
  (pad "7" thru_hole oval (at 15.24 0 180) (size 1.5 3) (drill 1) (layers "*.Cu" "*.Mask") (remove_unused_layers no) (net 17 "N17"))
  (pad "8" thru_hole oval (at 17.78 0 180) (size 1.5 3) (drill 1) (layers "*.Cu" "*.Mask") (remove_unused_layers no) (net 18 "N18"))
  (pad "9" thru_hole oval (at 20.32 0 180) (size 1.5 3) (drill 1) (layers "*.Cu" "*.Mask") (remove_unused_layers no) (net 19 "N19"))
  (pad "10" thru_hole oval (at 22.86 0 180) (size 1.5 3) (drill 1) (layers "*.Cu" "*.Mask") (remove_unused_layers no) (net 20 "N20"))
  (pad "11" thru_hole oval (at 25.4 0 180) (size 1.5 3) (drill 1) (layers "*.Cu" "*.Mask") (remove_unused_layers no) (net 9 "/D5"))
  (pad "12" thru_hole oval (at 27.94 0 180) (size 1.5 3) (drill 1) (layers "*.Cu" "*.Mask") (remove_unused_layers no) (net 10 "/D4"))
  (pad "13" thru_hole oval (at 30.48 0 180) (size 1.5 3) (drill 1) (layers "*.Cu" "*.Mask") (remove_unused_layers no) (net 11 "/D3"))
  (pad "14" thru_hole oval (at 33.02 0 180) (size 1.5 3) (drill 1) (layers "*.Cu" "*.Mask") (remove_unused_layers no) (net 12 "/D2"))
  (pad "15" thru_hole oval (at -2.54 0 180) (size 1.5 3) (drill 1) (layers "*.Cu" "*.Mask") (remove_unused_layers no) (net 16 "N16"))
  (pad "16" thru_hole oval (at -5.08 0 180) (size 1.5 3) (drill 1) (layers "*.Cu" "*.Mask") (remove_unused_layers no) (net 2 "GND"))
  (pad "A1" thru_hole rect (at -75.5 -14 180) (size 2 2) (drill 1) (layers "*.Cu" "*.Mask") (remove_unused_layers no) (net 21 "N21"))
  (pad "A2" thru_hole rect (at -75.5 -25 180) (size 2 2) (drill 1) (layers "*.Cu" "*.Mask") (remove_unused_layers no) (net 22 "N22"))
  (pad "K1" thru_hole rect (at -75.5 -18 180) (size 2 2) (drill 1) (layers "*.Cu" "*.Mask") (remove_unused_layers no) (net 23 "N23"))
  (pad "K2" thru_hole rect (at -75.5 -29 180) (size 2 2) (drill 1) (layers "*.Cu" "*.Mask") (remove_unused_layers no) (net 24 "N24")))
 (gr_line (start 134.62 83.82) (end 198.12 83.82) (stroke (width 0.1) (type solid)) (layer "Edge.Cuts"))
 (gr_line (start 134.62 111.76) (end 134.62 83.82) (stroke (width 0.1) (type solid)) (layer "Edge.Cuts"))
 (gr_line (start 198.12 111.76) (end 134.62 111.76) (stroke (width 0.1) (type solid)) (layer "Edge.Cuts"))
 (gr_line (start 198.12 83.82) (end 198.12 111.76) (stroke (width 0.1) (type solid)) (layer "Edge.Cuts"))
 (segment (start 187.96 101.6) (end 185.42 99.06) (width 0.25) (layer "F.Cu") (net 2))
 (segment (start 187.96 101.6) (end 193.04 101.6) (width 0.25) (layer "F.Cu") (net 2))
 (segment (start 172.72 101.6) (end 172.72 106.68) (width 0.25) (layer "F.Cu") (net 2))
 (segment (start 187.96 101.6) (end 185.42 104.14) (width 0.25) (layer "F.Cu") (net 2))
 (segment (start 185.42 104.14) (end 185.42 109.22) (width 0.25) (layer "F.Cu") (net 2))
 (segment (start 172.72 101.6) (end 165.1 101.6) (width 0.25) (layer "B.Cu") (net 2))
 (segment (start 157.48 88.9) (end 157.48 93.98) (width 0.25) (layer "B.Cu") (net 2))
 (segment (start 185.42 99.06) (end 180.34 99.06) (width 0.25) (layer "B.Cu") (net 2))
 (segment (start 180.34 99.06) (end 175.26 99.06) (width 0.25) (layer "B.Cu") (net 2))
 (segment (start 155.575 86.995) (end 157.48 88.9) (width 0.25) (layer "B.Cu") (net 2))
 (segment (start 145.495 87.075) (end 147.32 88.9) (width 0.25) (layer "B.Cu") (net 2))
 (segment (start 142.24 88.9) (end 144.065 87.075) (width 0.25) (layer "B.Cu") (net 2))
 (segment (start 139.78 96.6) (end 139.78 91.36) (width 0.25) (layer "B.Cu") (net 2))
 (segment (start 139.78 91.36) (end 142.24 88.9) (width 0.25) (layer "B.Cu") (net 2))
 (segment (start 144.065 87.075) (end 145.495 87.075) (width 0.25) (layer "B.Cu") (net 2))
 (segment (start 157.48 93.98) (end 165.1 101.6) (width 0.25) (layer "B.Cu") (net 2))
 (segment (start 149.225 86.995) (end 155.575 86.995) (width 0.25) (layer "B.Cu") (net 2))
 (segment (start 147.32 88.9) (end 149.225 86.995) (width 0.25) (layer "B.Cu") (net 2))
 (segment (start 175.26 99.06) (end 172.72 101.6) (width 0.25) (layer "B.Cu") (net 2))
 (segment (start 170.18 101.6) (end 172.72 99.06) (width 0.25) (layer "F.Cu") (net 3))
 (segment (start 170.18 106.68) (end 170.18 101.6) (width 0.25) (layer "F.Cu") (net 3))
 (segment (start 193.04 96.52) (end 185.42 96.52) (width 0.25) (layer "B.Cu") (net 3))
 (segment (start 180.34 96.52) (end 175.26 96.52) (width 0.25) (layer "B.Cu") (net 3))
 (segment (start 172.72 99.06) (end 165.1 99.06) (width 0.25) (layer "B.Cu") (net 3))
 (segment (start 185.42 96.52) (end 180.34 96.52) (width 0.25) (layer "B.Cu") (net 3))
 (segment (start 175.26 96.52) (end 172.72 99.06) (width 0.25) (layer "B.Cu") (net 3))
 (segment (start 156.21 100.33) (end 160.02 100.33) (width 0.25) (layer "B.Cu") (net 1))
 (segment (start 144.82 96.56) (end 139.78 101.6) (width 0.25) (layer "B.Cu") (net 1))
 (segment (start 154.94 101.6) (end 156.21 100.33) (width 0.25) (layer "B.Cu") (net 1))
 (segment (start 162.56 102.87) (end 171.45 102.87) (width 0.25) (layer "B.Cu") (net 1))
 (segment (start 149.86 88.9) (end 149.86 91.52) (width 0.25) (layer "B.Cu") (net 1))
 (segment (start 160.02 100.33) (end 162.56 102.87) (width 0.25) (layer "B.Cu") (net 1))
 (segment (start 144.82 96.56) (end 149.86 101.6) (width 0.25) (layer "B.Cu") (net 1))
 (segment (start 149.86 91.52) (end 144.82 96.56) (width 0.25) (layer "B.Cu") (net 1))
 (segment (start 154.94 101.6) (end 149.86 101.6) (width 0.25) (layer "B.Cu") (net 1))
 (segment (start 171.45 102.87) (end 175.26 106.68) (width 0.25) (layer "B.Cu") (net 1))
 (segment (start 149.5 93.98) (end 154.94 93.98) (width 0.25) (layer "F.Cu") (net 16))
 (segment (start 144.78 88.9) (end 144.78 89.26) (width 0.25) (layer "F.Cu") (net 16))
 (segment (start 144.78 89.26) (end 149.5 93.98) (width 0.25) (layer "F.Cu") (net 16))
 (segment (start 152.36 96.52) (end 152.4 96.52) (width 0.25) (layer "B.Cu") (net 13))
 (segment (start 152.4 96.52) (end 152.4 88.9) (width 0.25) (layer "B.Cu") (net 13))
 (segment (start 149.78 99.1) (end 152.36 96.52) (width 0.25) (layer "B.Cu") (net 13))
 (segment (start 157.48 106.68) (end 158.75 107.95) (width 0.25) (layer "B.Cu") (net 8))
 (segment (start 186.69 107.95) (end 187.96 109.22) (width 0.25) (layer "B.Cu") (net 8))
 (segment (start 158.75 107.95) (end 186.69 107.95) (width 0.25) (layer "B.Cu") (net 8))
 (segment (start 144.78 104.14) (end 154.94 104.14) (width 0.25) (layer "B.Cu") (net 4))
 (segment (start 157.48 101.6) (end 160.02 104.14) (width 0.25) (layer "B.Cu") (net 4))
 (segment (start 165.1 104.14) (end 167.64 106.68) (width 0.25) (layer "B.Cu") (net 4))
 (segment (start 160.02 104.14) (end 165.1 104.14) (width 0.25) (layer "B.Cu") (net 4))
 (segment (start 142.24 106.68) (end 144.78 104.14) (width 0.25) (layer "B.Cu") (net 4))
 (segment (start 154.94 104.14) (end 157.48 101.6) (width 0.25) (layer "B.Cu") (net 4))
 (segment (start 176.53 110.49) (end 151.13 110.49) (width 0.25) (layer "F.Cu") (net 12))
 (segment (start 151.13 110.49) (end 147.32 106.68) (width 0.25) (layer "F.Cu") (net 12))
 (segment (start 178.25 90.99) (end 178.25 108.77) (width 0.25) (layer "F.Cu") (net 12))
 (segment (start 180.34 88.9) (end 178.25 90.99) (width 0.25) (layer "F.Cu") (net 12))
 (segment (start 178.25 108.77) (end 176.53 110.49) (width 0.25) (layer "F.Cu") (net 12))
 (segment (start 177.8 108.32) (end 176.08 110.04) (width 0.25) (layer "F.Cu") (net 11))
 (segment (start 177.8 88.9) (end 177.8 108.32) (width 0.25) (layer "F.Cu") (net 11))
 (segment (start 153.22 110.04) (end 176.08 110.04) (width 0.25) (layer "F.Cu") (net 11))
 (segment (start 149.86 106.68) (end 153.22 110.04) (width 0.25) (layer "F.Cu") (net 11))
 (segment (start 154.94 109.22) (end 176.16 109.22) (width 0.25) (layer "F.Cu") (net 10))
 (segment (start 152.4 106.68) (end 154.94 109.22) (width 0.25) (layer "F.Cu") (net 10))
 (segment (start 176.98 90.62) (end 175.26 88.9) (width 0.25) (layer "F.Cu") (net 10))
 (segment (start 176.98 108.4) (end 176.98 90.62) (width 0.25) (layer "F.Cu") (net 10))
 (segment (start 176.16 109.22) (end 176.98 108.4) (width 0.25) (layer "F.Cu") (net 10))
 (segment (start 154.94 106.68) (end 157.03 108.77) (width 0.25) (layer "F.Cu") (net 9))
 (segment (start 157.03 108.77) (end 175.71 108.77) (width 0.25) (layer "F.Cu") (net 9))
 (segment (start 176.53 107.95) (end 176.53 92.71) (width 0.25) (layer "F.Cu") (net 9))
 (segment (start 172.72 88.9) (end 176.53 92.71) (width 0.25) (layer "F.Cu") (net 9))
 (segment (start 175.71 108.77) (end 176.53 107.95) (width 0.25) (layer "F.Cu") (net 9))
 (segment (start 140.97 105.41) (end 158.75 105.41) (width 0.25) (layer "F.Cu") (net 7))
 (segment (start 139.7 106.68) (end 140.97 105.41) (width 0.25) (layer "F.Cu") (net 7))
 (segment (start 158.75 105.41) (end 160.02 106.68) (width 0.25) (layer "F.Cu") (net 7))
 (segment (start 160.02 104.14) (end 162.56 106.68) (width 0.25) (layer "F.Cu") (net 6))
 (segment (start 160.02 88.9) (end 160.02 104.14) (width 0.25) (layer "F.Cu") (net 6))
 (segment (start 163.68 105.26) (end 165.1 106.68) (width 0.25) (layer "F.Cu") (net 5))
 (segment (start 162.56 86.36) (end 157.48 86.36) (width 0.25) (layer "F.Cu") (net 5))
 (segment (start 157.48 86.36) (end 154.94 88.9) (width 0.25) (layer "F.Cu") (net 5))
 (segment (start 163.68 87.48) (end 163.68 105.26) (width 0.25) (layer "F.Cu") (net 5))
 (segment (start 163.68 87.48) (end 162.56 86.36) (width 0.25) (layer "F.Cu") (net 5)))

